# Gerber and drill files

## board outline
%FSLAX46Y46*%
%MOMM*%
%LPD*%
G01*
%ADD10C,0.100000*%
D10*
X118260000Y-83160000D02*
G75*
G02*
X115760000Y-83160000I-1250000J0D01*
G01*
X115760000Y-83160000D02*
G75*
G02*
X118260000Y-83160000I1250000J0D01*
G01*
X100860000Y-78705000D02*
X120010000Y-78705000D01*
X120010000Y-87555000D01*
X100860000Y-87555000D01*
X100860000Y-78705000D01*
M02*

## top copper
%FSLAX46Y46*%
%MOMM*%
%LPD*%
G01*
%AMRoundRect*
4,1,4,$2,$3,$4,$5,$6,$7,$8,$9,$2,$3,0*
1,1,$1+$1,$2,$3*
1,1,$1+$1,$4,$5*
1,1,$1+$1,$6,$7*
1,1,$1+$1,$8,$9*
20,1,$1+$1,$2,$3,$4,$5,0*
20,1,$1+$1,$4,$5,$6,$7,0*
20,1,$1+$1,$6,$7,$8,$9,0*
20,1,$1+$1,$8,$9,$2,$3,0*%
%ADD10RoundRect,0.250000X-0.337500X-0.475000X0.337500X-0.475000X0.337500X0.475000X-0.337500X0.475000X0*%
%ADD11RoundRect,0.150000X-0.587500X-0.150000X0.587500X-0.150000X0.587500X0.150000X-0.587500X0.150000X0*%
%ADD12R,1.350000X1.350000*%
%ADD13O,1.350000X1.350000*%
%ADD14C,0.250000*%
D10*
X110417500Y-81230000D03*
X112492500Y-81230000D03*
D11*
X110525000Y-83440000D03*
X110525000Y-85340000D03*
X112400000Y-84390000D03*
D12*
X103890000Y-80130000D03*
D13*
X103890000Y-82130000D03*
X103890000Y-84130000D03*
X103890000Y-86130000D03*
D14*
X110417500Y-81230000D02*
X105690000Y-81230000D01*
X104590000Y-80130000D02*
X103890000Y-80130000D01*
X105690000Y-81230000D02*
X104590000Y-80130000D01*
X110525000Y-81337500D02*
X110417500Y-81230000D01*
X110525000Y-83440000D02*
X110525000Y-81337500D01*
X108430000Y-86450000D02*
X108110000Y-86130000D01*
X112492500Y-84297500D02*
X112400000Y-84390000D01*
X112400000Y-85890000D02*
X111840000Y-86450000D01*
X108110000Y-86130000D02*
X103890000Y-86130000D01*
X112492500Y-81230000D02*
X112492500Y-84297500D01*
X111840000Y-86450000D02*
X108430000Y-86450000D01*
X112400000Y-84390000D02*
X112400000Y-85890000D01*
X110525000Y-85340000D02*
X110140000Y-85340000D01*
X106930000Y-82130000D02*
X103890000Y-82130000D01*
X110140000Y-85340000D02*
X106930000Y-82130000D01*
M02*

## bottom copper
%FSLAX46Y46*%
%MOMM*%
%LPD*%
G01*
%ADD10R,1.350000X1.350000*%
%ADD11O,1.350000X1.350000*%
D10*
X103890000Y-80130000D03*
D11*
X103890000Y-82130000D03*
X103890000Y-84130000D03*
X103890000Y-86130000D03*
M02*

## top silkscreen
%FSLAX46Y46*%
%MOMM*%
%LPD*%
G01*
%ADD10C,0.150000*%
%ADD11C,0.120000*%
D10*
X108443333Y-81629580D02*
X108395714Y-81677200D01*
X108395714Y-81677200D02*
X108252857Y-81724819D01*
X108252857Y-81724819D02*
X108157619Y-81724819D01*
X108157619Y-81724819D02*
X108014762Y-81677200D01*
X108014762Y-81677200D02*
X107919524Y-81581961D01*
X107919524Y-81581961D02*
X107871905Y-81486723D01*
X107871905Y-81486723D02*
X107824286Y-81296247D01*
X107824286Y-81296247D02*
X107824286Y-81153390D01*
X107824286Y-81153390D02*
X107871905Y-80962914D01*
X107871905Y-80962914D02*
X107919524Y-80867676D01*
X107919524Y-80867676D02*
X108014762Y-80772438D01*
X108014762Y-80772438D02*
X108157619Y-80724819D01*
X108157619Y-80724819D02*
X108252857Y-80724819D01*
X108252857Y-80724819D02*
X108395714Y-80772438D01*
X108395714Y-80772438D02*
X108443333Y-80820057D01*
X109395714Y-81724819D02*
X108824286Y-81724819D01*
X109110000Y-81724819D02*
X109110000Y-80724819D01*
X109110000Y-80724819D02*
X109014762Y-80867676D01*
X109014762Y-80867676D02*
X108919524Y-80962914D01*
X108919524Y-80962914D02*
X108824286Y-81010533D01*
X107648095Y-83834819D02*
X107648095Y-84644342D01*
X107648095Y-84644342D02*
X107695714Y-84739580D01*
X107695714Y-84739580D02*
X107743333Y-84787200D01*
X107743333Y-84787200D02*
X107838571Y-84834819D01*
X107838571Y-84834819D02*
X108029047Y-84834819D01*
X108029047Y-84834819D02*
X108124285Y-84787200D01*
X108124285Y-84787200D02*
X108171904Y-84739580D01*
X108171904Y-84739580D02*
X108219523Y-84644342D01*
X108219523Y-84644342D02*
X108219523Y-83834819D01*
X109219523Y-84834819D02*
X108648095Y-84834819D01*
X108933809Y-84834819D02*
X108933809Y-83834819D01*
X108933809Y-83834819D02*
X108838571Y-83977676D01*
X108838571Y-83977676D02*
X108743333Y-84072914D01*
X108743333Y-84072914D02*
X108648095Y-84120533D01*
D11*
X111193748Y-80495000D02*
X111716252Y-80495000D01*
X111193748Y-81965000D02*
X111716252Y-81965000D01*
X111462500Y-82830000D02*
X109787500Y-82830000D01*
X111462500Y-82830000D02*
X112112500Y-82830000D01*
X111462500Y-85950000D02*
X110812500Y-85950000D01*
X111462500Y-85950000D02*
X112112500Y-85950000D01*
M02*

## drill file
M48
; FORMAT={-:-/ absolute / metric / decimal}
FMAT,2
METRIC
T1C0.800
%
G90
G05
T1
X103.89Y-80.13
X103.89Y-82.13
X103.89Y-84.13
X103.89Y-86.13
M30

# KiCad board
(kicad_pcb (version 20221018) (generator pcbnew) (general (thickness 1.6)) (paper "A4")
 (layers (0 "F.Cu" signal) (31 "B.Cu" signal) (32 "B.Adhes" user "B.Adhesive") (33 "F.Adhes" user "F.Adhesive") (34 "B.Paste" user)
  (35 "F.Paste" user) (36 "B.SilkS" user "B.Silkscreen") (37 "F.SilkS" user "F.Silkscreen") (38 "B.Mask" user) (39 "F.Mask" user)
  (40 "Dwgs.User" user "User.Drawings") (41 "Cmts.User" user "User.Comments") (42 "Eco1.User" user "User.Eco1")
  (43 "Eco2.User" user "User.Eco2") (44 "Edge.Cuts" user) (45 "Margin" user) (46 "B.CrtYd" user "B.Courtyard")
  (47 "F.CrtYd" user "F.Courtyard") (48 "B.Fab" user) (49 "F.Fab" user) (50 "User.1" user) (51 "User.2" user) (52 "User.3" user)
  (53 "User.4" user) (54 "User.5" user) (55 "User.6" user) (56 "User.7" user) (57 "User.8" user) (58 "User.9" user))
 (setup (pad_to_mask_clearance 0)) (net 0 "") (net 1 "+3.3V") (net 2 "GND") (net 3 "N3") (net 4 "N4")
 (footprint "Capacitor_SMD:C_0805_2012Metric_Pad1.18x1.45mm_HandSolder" (layer "F.Cu") (at 111.455 81.23)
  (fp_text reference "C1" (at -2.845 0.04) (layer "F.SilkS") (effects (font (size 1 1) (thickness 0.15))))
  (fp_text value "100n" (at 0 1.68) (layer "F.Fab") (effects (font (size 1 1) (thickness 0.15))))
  (fp_line (start -0.261252 -0.735) (end 0.261252 -0.735) (stroke (width 0.12) (type solid)) (layer "F.SilkS"))
  (fp_line (start -0.261252 0.735) (end 0.261252 0.735) (stroke (width 0.12) (type solid)) (layer "F.SilkS"))
  (pad "1" smd roundrect (at -1.0375 0) (size 1.175 1.45) (layers "F.Cu" "F.Paste" "F.Mask") (roundrect_rratio 0.2127659574) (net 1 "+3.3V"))
  (pad "2" smd roundrect (at 1.0375 0) (size 1.175 1.45) (layers "F.Cu" "F.Paste" "F.Mask") (roundrect_rratio 0.2127659574) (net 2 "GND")))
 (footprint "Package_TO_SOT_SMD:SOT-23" (layer "F.Cu") (at 111.4625 84.39)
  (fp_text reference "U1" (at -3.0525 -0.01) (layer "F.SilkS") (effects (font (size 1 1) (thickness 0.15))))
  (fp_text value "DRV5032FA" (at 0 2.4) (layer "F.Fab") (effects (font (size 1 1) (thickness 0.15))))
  (fp_line (start 0 -1.56) (end -1.675 -1.56) (stroke (width 0.12) (type solid)) (layer "F.SilkS"))
  (fp_line (start 0 -1.56) (end 0.65 -1.56) (stroke (width 0.12) (type solid)) (layer "F.SilkS"))
  (fp_line (start 0 1.56) (end -0.65 1.56) (stroke (width 0.12) (type solid)) (layer "F.SilkS"))
  (fp_line (start 0 1.56) (end 0.65 1.56) (stroke (width 0.12) (type solid)) (layer "F.SilkS"))
  (pad "1" smd roundrect (at -0.9375 -0.95) (size 1.475 0.6) (layers "F.Cu" "F.Paste" "F.Mask") (roundrect_rratio 0.25) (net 1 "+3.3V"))
  (pad "2" smd roundrect (at -0.9375 0.95) (size 1.475 0.6) (layers "F.Cu" "F.Paste" "F.Mask") (roundrect_rratio 0.25) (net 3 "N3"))
  (pad "3" smd roundrect (at 0.9375 0) (size 1.475 0.6) (layers "F.Cu" "F.Paste" "F.Mask") (roundrect_rratio 0.25) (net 2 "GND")))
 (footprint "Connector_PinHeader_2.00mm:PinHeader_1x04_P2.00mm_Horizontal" (layer "B.Cu") (at 103.89 80.13 180)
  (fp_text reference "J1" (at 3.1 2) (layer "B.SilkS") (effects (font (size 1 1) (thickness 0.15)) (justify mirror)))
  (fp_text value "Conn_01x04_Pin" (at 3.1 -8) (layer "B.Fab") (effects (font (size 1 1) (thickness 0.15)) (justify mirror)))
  (pad "1" thru_hole rect (at 0 0 180) (size 1.35 1.35) (drill 0.8) (layers "*.Cu" "*.Mask") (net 1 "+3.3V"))
  (pad "2" thru_hole oval (at 0 -2 180) (size 1.35 1.35) (drill 0.8) (layers "*.Cu" "*.Mask") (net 3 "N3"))
  (pad "3" thru_hole oval (at 0 -4 180) (size 1.35 1.35) (drill 0.8) (layers "*.Cu" "*.Mask") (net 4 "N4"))
  (pad "4" thru_hole oval (at 0 -6 180) (size 1.35 1.35) (drill 0.8) (layers "*.Cu" "*.Mask") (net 2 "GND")))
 (gr_circle (center 117.01 83.16) (end 118.26 83.16) (stroke (width 0.1) (type default)) (fill none) (layer "Edge.Cuts"))
 (gr_rect (start 100.86 78.705) (end 120.01 87.555) (stroke (width 0.1) (type default)) (fill none) (layer "Edge.Cuts"))
 (segment (start 110.4175 81.23) (end 105.69 81.23) (width 0.25) (layer "F.Cu") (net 1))
 (segment (start 104.59 80.13) (end 103.89 80.13) (width 0.25) (layer "F.Cu") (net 1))
 (segment (start 105.69 81.23) (end 104.59 80.13) (width 0.25) (layer "F.Cu") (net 1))
 (segment (start 110.525 81.3375) (end 110.4175 81.23) (width 0.25) (layer "F.Cu") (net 1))
 (segment (start 110.525 83.44) (end 110.525 81.3375) (width 0.25) (layer "F.Cu") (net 1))
 (segment (start 108.43 86.45) (end 108.11 86.13) (width 0.25) (layer "F.Cu") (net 2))
 (segment (start 112.4925 84.2975) (end 112.4 84.39) (width 0.25) (layer "F.Cu") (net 2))
 (segment (start 112.4 85.89) (end 111.84 86.45) (width 0.25) (layer "F.Cu") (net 2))
 (segment (start 108.11 86.13) (end 103.89 86.13) (width 0.25) (layer "F.Cu") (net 2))
 (segment (start 112.4925 81.23) (end 112.4925 84.2975) (width 0.25) (layer "F.Cu") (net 2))
 (segment (start 111.84 86.45) (end 108.43 86.45) (width 0.25) (layer "F.Cu") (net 2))
 (segment (start 112.4 84.39) (end 112.4 85.89) (width 0.25) (layer "F.Cu") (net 2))
 (segment (start 110.525 85.34) (end 110.14 85.34) (width 0.25) (layer "F.Cu") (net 3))
 (segment (start 106.93 82.13) (end 103.89 82.13) (width 0.25) (layer "F.Cu") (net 3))
 (segment (start 110.14 85.34) (end 106.93 82.13) (width 0.25) (layer "F.Cu") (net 3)))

